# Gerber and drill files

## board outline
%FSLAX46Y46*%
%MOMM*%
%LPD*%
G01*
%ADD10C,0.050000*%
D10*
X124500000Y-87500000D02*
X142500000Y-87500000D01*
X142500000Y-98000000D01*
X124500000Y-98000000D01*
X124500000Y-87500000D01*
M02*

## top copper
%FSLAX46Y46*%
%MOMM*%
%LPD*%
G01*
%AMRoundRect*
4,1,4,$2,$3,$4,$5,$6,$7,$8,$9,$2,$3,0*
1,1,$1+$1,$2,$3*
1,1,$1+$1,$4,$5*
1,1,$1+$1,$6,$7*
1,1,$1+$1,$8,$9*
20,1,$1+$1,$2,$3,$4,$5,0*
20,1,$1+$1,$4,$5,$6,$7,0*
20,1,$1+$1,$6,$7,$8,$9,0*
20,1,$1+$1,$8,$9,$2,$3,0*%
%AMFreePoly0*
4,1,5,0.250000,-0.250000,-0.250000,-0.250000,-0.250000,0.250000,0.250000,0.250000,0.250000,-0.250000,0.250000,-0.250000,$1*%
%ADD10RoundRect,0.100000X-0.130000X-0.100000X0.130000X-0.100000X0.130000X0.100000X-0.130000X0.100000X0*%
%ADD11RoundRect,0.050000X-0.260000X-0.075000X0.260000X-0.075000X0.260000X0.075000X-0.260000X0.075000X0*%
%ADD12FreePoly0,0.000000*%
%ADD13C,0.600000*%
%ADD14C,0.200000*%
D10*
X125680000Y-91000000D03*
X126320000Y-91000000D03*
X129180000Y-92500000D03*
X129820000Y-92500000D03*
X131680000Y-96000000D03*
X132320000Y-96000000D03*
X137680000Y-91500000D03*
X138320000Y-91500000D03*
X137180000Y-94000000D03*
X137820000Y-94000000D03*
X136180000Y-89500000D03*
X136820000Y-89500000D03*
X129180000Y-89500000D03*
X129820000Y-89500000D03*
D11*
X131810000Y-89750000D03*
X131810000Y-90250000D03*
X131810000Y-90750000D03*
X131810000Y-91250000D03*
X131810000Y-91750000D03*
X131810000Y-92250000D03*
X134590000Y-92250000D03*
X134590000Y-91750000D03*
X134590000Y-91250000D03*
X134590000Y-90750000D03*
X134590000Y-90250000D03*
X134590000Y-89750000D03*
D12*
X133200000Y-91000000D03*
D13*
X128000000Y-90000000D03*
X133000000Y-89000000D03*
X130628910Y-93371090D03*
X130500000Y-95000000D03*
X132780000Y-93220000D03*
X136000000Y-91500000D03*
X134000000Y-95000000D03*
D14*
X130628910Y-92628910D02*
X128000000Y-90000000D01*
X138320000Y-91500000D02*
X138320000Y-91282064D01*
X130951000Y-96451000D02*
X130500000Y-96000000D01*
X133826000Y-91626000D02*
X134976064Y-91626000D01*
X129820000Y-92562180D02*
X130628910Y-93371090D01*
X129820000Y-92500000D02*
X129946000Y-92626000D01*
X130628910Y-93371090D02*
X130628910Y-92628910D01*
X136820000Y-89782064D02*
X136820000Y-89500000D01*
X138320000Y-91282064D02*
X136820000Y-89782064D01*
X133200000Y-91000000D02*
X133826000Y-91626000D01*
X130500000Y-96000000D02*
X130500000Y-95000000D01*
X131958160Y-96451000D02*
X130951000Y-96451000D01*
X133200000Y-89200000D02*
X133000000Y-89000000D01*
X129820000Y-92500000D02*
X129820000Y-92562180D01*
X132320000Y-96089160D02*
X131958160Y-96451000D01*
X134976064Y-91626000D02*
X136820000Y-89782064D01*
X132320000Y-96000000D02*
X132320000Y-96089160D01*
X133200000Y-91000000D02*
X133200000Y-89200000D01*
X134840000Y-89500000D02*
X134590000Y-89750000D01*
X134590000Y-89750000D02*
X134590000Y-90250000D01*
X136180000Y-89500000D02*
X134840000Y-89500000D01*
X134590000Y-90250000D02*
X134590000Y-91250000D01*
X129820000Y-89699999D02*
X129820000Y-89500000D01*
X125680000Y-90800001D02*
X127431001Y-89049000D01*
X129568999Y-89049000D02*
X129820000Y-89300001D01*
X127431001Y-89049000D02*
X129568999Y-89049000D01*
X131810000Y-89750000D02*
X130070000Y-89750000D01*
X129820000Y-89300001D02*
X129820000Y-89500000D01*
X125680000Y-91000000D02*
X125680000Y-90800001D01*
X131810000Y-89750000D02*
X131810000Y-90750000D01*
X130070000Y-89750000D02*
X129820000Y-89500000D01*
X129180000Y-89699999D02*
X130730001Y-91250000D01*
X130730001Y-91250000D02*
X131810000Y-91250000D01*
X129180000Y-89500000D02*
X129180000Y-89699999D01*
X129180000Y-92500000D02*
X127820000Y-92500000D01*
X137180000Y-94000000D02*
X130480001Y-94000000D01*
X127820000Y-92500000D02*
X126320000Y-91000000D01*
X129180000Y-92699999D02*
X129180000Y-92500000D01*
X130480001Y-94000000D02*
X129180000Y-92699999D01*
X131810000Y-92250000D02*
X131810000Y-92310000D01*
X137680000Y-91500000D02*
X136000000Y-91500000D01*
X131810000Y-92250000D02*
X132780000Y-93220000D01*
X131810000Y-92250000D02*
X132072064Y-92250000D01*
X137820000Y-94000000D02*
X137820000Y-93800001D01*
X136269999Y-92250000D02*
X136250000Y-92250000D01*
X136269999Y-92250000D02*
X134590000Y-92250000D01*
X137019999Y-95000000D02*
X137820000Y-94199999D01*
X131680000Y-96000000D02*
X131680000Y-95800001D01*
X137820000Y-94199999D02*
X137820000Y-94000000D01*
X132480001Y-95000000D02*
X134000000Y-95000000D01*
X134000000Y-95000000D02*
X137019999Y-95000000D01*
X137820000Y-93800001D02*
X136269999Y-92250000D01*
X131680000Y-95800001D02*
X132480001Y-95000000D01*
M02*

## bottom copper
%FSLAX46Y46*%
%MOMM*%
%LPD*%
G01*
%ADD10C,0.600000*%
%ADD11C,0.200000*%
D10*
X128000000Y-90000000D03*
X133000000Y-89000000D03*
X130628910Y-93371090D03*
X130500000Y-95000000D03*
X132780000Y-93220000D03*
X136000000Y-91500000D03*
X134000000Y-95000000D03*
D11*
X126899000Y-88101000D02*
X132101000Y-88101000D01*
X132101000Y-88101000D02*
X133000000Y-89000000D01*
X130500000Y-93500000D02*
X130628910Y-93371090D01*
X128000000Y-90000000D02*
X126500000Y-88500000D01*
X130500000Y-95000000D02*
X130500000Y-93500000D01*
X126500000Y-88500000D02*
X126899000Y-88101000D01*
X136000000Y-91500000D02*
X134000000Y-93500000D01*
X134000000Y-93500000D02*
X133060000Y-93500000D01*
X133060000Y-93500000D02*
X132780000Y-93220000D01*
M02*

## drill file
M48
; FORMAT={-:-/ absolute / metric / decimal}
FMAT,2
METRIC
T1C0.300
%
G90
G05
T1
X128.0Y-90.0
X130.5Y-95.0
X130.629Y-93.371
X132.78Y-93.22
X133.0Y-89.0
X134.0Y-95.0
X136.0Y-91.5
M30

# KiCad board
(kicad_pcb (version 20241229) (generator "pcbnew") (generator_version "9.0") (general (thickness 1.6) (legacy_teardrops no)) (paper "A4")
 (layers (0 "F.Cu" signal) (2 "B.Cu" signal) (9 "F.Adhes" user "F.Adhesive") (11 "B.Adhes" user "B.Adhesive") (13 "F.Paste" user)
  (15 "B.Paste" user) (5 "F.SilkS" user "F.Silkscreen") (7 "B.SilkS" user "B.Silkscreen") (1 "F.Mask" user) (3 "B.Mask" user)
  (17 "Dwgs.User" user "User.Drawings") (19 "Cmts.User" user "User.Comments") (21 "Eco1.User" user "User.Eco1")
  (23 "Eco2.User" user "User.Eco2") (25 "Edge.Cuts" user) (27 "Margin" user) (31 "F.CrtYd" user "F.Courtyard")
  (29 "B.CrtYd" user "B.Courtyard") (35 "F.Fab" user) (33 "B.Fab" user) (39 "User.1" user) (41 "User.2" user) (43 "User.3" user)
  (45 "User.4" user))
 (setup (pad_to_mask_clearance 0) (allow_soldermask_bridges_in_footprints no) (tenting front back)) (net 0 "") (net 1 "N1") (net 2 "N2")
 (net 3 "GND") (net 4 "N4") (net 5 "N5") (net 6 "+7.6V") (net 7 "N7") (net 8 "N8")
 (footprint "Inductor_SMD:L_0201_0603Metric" (layer "F.Cu") (at 126 91)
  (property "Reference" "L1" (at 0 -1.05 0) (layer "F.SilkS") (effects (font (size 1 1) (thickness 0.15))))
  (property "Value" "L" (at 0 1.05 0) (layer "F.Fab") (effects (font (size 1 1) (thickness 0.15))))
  (pad "" smd roundrect (at -0.345 0) (size 0.318 0.36) (layers "F.Paste") (roundrect_rratio 0.25))
  (pad "" smd roundrect (at 0.345 0) (size 0.318 0.36) (layers "F.Paste") (roundrect_rratio 0.25))
  (pad "1" smd roundrect (at -0.32 0) (size 0.46 0.4) (layers "F.Cu" "F.Mask") (roundrect_rratio 0.25) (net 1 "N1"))
  (pad "2" smd roundrect (at 0.32 0) (size 0.46 0.4) (layers "F.Cu" "F.Mask") (roundrect_rratio 0.25) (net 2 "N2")))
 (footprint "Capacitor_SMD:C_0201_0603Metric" (layer "F.Cu") (at 129.5 92.5)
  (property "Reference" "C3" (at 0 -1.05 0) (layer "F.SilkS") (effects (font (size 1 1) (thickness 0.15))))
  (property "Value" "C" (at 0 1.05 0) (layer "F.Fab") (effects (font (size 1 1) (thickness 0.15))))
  (pad "" smd roundrect (at -0.345 0) (size 0.318 0.36) (layers "F.Paste") (roundrect_rratio 0.25))
  (pad "" smd roundrect (at 0.345 0) (size 0.318 0.36) (layers "F.Paste") (roundrect_rratio 0.25))
  (pad "1" smd roundrect (at -0.32 0) (size 0.46 0.4) (layers "F.Cu" "F.Mask") (roundrect_rratio 0.25) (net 2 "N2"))
  (pad "2" smd roundrect (at 0.32 0) (size 0.46 0.4) (layers "F.Cu" "F.Mask") (roundrect_rratio 0.25) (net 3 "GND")))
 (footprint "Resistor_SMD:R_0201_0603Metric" (layer "F.Cu") (at 132 96)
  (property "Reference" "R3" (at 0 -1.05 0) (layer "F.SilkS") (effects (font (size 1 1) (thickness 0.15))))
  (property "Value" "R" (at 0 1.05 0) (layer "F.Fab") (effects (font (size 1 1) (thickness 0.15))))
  (pad "" smd roundrect (at -0.345 0) (size 0.318 0.36) (layers "F.Paste") (roundrect_rratio 0.25))
  (pad "" smd roundrect (at 0.345 0) (size 0.318 0.36) (layers "F.Paste") (roundrect_rratio 0.25))
  (pad "1" smd roundrect (at -0.32 0) (size 0.46 0.4) (layers "F.Cu" "F.Mask") (roundrect_rratio 0.25) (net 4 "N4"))
  (pad "2" smd roundrect (at 0.32 0) (size 0.46 0.4) (layers "F.Cu" "F.Mask") (roundrect_rratio 0.25) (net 3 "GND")))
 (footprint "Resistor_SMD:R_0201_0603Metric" (layer "F.Cu") (at 138 91.5)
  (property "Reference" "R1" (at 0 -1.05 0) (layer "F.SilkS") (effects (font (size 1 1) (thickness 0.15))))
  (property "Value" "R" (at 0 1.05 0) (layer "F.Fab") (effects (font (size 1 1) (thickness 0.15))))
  (pad "" smd roundrect (at -0.345 0) (size 0.318 0.36) (layers "F.Paste") (roundrect_rratio 0.25))
  (pad "" smd roundrect (at 0.345 0) (size 0.318 0.36) (layers "F.Paste") (roundrect_rratio 0.25))
  (pad "1" smd roundrect (at -0.32 0) (size 0.46 0.4) (layers "F.Cu" "F.Mask") (roundrect_rratio 0.25) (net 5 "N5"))
  (pad "2" smd roundrect (at 0.32 0) (size 0.46 0.4) (layers "F.Cu" "F.Mask") (roundrect_rratio 0.25) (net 3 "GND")))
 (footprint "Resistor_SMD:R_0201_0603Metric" (layer "F.Cu") (at 137.5 94)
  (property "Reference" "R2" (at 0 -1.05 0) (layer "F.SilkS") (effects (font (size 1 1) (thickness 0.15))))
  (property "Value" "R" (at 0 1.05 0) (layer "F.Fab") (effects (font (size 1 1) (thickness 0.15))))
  (pad "" smd roundrect (at -0.345 0) (size 0.318 0.36) (layers "F.Paste") (roundrect_rratio 0.25))
  (pad "" smd roundrect (at 0.345 0) (size 0.318 0.36) (layers "F.Paste") (roundrect_rratio 0.25))
  (pad "1" smd roundrect (at -0.32 0) (size 0.46 0.4) (layers "F.Cu" "F.Mask") (roundrect_rratio 0.25) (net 2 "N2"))
  (pad "2" smd roundrect (at 0.32 0) (size 0.46 0.4) (layers "F.Cu" "F.Mask") (roundrect_rratio 0.25) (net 4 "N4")))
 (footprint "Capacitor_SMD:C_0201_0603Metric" (layer "F.Cu") (at 136.5 89.5)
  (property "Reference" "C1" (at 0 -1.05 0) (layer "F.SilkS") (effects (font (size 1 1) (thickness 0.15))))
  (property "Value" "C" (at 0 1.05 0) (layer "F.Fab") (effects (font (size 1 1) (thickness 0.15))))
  (pad "" smd roundrect (at -0.345 0) (size 0.318 0.36) (layers "F.Paste") (roundrect_rratio 0.25))
  (pad "" smd roundrect (at 0.345 0) (size 0.318 0.36) (layers "F.Paste") (roundrect_rratio 0.25))
  (pad "1" smd roundrect (at -0.32 0) (size 0.46 0.4) (layers "F.Cu" "F.Mask") (roundrect_rratio 0.25) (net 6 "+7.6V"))
  (pad "2" smd roundrect (at 0.32 0) (size 0.46 0.4) (layers "F.Cu" "F.Mask") (roundrect_rratio 0.25) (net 3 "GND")))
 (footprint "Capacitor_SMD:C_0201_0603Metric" (layer "F.Cu") (at 129.5 89.5)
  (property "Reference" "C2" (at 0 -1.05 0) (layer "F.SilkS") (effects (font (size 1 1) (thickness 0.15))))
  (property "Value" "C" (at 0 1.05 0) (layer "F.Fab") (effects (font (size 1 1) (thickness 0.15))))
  (pad "" smd roundrect (at -0.345 0) (size 0.318 0.36) (layers "F.Paste") (roundrect_rratio 0.25))
  (pad "" smd roundrect (at 0.345 0) (size 0.318 0.36) (layers "F.Paste") (roundrect_rratio 0.25))
  (pad "1" smd roundrect (at -0.32 0) (size 0.46 0.4) (layers "F.Cu" "F.Mask") (roundrect_rratio 0.25) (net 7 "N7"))
  (pad "2" smd roundrect (at 0.32 0) (size 0.46 0.4) (layers "F.Cu" "F.Mask") (roundrect_rratio 0.25) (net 1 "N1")))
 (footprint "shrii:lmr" (layer "F.Cu") (at 139.5 94)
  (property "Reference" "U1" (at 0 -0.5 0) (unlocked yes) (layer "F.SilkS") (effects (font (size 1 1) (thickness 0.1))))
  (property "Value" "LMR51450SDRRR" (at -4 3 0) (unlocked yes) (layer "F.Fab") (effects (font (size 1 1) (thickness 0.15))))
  (pad "1" smd roundrect (at -7.69 -4.25) (size 0.62 0.25) (layers "F.Cu" "F.Paste") (roundrect_rratio 0.2) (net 1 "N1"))
  (pad "2" smd roundrect (at -7.69 -3.75) (size 0.62 0.25) (layers "F.Cu" "F.Paste") (roundrect_rratio 0.2) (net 1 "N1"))
  (pad "3" smd roundrect (at -7.69 -3.25) (size 0.62 0.25) (layers "F.Cu" "F.Paste") (roundrect_rratio 0.2) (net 1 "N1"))
  (pad "4" smd roundrect (at -7.69 -2.75) (size 0.62 0.25) (layers "F.Cu" "F.Paste") (roundrect_rratio 0.2) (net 7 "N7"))
  (pad "5" smd roundrect (at -7.69 -2.25) (size 0.62 0.25) (layers "F.Cu" "F.Paste") (roundrect_rratio 0.2) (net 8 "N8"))
  (pad "6" smd roundrect (at -7.69 -1.75) (size 0.62 0.25) (layers "F.Cu" "F.Paste") (roundrect_rratio 0.2) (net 5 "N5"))
  (pad "7" smd roundrect (at -4.91 -1.75) (size 0.62 0.25) (layers "F.Cu" "F.Paste") (roundrect_rratio 0.2) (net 4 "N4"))
  (pad "8" smd roundrect (at -4.91 -2.25) (size 0.62 0.25) (layers "F.Cu" "F.Paste") (roundrect_rratio 0.2) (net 3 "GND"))
  (pad "9" smd roundrect (at -4.91 -2.75) (size 0.62 0.25) (layers "F.Cu" "F.Paste") (roundrect_rratio 0.2) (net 6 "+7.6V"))
  (pad "10" smd roundrect (at -4.91 -3.25) (size 0.62 0.25) (layers "F.Cu" "F.Paste") (roundrect_rratio 0.2) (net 6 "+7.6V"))
  (pad "11" smd roundrect (at -4.91 -3.75) (size 0.62 0.25) (layers "F.Cu" "F.Paste") (roundrect_rratio 0.2) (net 6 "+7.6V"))
  (pad "12" smd roundrect (at -4.91 -4.25) (size 0.62 0.25) (layers "F.Cu" "F.Paste") (roundrect_rratio 0.2) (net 6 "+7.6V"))
  (pad "13" smd custom (at -6.3 -3) (size 0.5 0.5) (layers "F.Cu") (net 3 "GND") (zone_connect 2)
   (options (clearance outline) (anchor rect)) (primitives)))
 (gr_rect (start 124.5 87.5) (end 142.5 98) (stroke (width 0.05) (type default)) (fill no) (layer "Edge.Cuts"))
 (segment (start 130.62891 92.62891) (end 128 90) (width 0.2) (layer "F.Cu") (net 3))
 (segment (start 138.32 91.5) (end 138.32 91.282064) (width 0.2) (layer "F.Cu") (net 3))
 (segment (start 130.951 96.451) (end 130.5 96) (width 0.2) (layer "F.Cu") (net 3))
 (segment (start 133.826 91.626) (end 134.976064 91.626) (width 0.2) (layer "F.Cu") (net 3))
 (segment (start 129.82 92.56218) (end 130.62891 93.37109) (width 0.2) (layer "F.Cu") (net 3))
 (segment (start 129.82 92.5) (end 129.946 92.626) (width 0.2) (layer "F.Cu") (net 3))
 (segment (start 130.62891 93.37109) (end 130.62891 92.62891) (width 0.2) (layer "F.Cu") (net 3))
 (segment (start 136.82 89.782064) (end 136.82 89.5) (width 0.2) (layer "F.Cu") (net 3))
 (segment (start 138.32 91.282064) (end 136.82 89.782064) (width 0.2) (layer "F.Cu") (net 3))
 (segment (start 133.2 91) (end 133.826 91.626) (width 0.2) (layer "F.Cu") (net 3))
 (segment (start 130.5 96) (end 130.5 95) (width 0.2) (layer "F.Cu") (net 3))
 (segment (start 131.95816 96.451) (end 130.951 96.451) (width 0.2) (layer "F.Cu") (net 3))
 (segment (start 133.2 89.2) (end 133 89) (width 0.2) (layer "F.Cu") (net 3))
 (segment (start 129.82 92.5) (end 129.82 92.56218) (width 0.2) (layer "F.Cu") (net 3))
 (segment (start 132.32 96.08916) (end 131.95816 96.451) (width 0.2) (layer "F.Cu") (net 3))
 (segment (start 134.976064 91.626) (end 136.82 89.782064) (width 0.2) (layer "F.Cu") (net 3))
 (segment (start 132.32 96) (end 132.32 96.08916) (width 0.2) (layer "F.Cu") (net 3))
 (segment (start 133.2 91) (end 133.2 89.2) (width 0.2) (layer "F.Cu") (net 3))
 (via (at 128 90) (size 0.6) (drill 0.3) (layers "F.Cu" "B.Cu") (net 3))
 (via (at 133 89) (size 0.6) (drill 0.3) (layers "F.Cu" "B.Cu") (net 3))
 (via (at 130.62891 93.37109) (size 0.6) (drill 0.3) (layers "F.Cu" "B.Cu") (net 3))
 (via (at 130.5 95) (size 0.6) (drill 0.3) (layers "F.Cu" "B.Cu") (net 3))
 (segment (start 126.899 88.101) (end 132.101 88.101) (width 0.2) (layer "B.Cu") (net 3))
 (segment (start 132.101 88.101) (end 133 89) (width 0.2) (layer "B.Cu") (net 3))
 (segment (start 130.5 93.5) (end 130.62891 93.37109) (width 0.2) (layer "B.Cu") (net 3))
 (segment (start 128 90) (end 126.5 88.5) (width 0.2) (layer "B.Cu") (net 3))
 (segment (start 130.5 95) (end 130.5 93.5) (width 0.2) (layer "B.Cu") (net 3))
 (segment (start 126.5 88.5) (end 126.899 88.101) (width 0.2) (layer "B.Cu") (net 3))
 (segment (start 134.84 89.5) (end 134.59 89.75) (width 0.2) (layer "F.Cu") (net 6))
 (segment (start 134.59 89.75) (end 134.59 90.25) (width 0.2) (layer "F.Cu") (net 6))
 (segment (start 136.18 89.5) (end 134.84 89.5) (width 0.2) (layer "F.Cu") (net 6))
 (segment (start 134.59 90.25) (end 134.59 91.25) (width 0.2) (layer "F.Cu") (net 6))
 (segment (start 129.82 89.699999) (end 129.82 89.5) (width 0.2) (layer "F.Cu") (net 1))
 (segment (start 125.68 90.800001) (end 127.431001 89.049) (width 0.2) (layer "F.Cu") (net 1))
 (segment (start 129.568999 89.049) (end 129.82 89.300001) (width 0.2) (layer "F.Cu") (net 1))
 (segment (start 127.431001 89.049) (end 129.568999 89.049) (width 0.2) (layer "F.Cu") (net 1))
 (segment (start 131.81 89.75) (end 130.07 89.75) (width 0.2) (layer "F.Cu") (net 1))
 (segment (start 129.82 89.300001) (end 129.82 89.5) (width 0.2) (layer "F.Cu") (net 1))
 (segment (start 125.68 91) (end 125.68 90.800001) (width 0.2) (layer "F.Cu") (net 1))
 (segment (start 131.81 89.75) (end 131.81 90.75) (width 0.2) (layer "F.Cu") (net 1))
 (segment (start 130.07 89.75) (end 129.82 89.5) (width 0.2) (layer "F.Cu") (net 1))
 (segment (start 129.18 89.699999) (end 130.730001 91.25) (width 0.2) (layer "F.Cu") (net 7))
 (segment (start 130.730001 91.25) (end 131.81 91.25) (width 0.2) (layer "F.Cu") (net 7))
 (segment (start 129.18 89.5) (end 129.18 89.699999) (width 0.2) (layer "F.Cu") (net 7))
 (segment (start 129.18 92.5) (end 127.82 92.5) (width 0.2) (layer "F.Cu") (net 2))
 (segment (start 137.18 94) (end 130.480001 94) (width 0.2) (layer "F.Cu") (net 2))
 (segment (start 127.82 92.5) (end 126.32 91) (width 0.2) (layer "F.Cu") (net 2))
 (segment (start 129.18 92.699999) (end 129.18 92.5) (width 0.2) (layer "F.Cu") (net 2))
 (segment (start 130.480001 94) (end 129.18 92.699999) (width 0.2) (layer "F.Cu") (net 2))
 (segment (start 131.81 92.25) (end 131.81 92.31) (width 0.2) (layer "F.Cu") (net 5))
 (segment (start 137.68 91.5) (end 136 91.5) (width 0.2) (layer "F.Cu") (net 5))
 (segment (start 131.81 92.25) (end 132.78 93.22) (width 0.2) (layer "F.Cu") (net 5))
 (segment (start 131.81 92.25) (end 132.072064 92.25) (width 0.2) (layer "F.Cu") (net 5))
 (via (at 132.78 93.22) (size 0.6) (drill 0.3) (layers "F.Cu" "B.Cu") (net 5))
 (via (at 136 91.5) (size 0.6) (drill 0.3) (layers "F.Cu" "B.Cu") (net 5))
 (segment (start 136 91.5) (end 134 93.5) (width 0.2) (layer "B.Cu") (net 5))
 (segment (start 134 93.5) (end 133.06 93.5) (width 0.2) (layer "B.Cu") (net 5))
 (segment (start 133.06 93.5) (end 132.78 93.22) (width 0.2) (layer "B.Cu") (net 5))
 (segment (start 137.82 94) (end 137.82 93.800001) (width 0.2) (layer "F.Cu") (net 4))
 (segment (start 136.269999 92.25) (end 136.25 92.25) (width 0.2) (layer "F.Cu") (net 4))
 (segment (start 136.269999 92.25) (end 134.59 92.25) (width 0.2) (layer "F.Cu") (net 4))
 (segment (start 137.019999 95) (end 137.82 94.199999) (width 0.2) (layer "F.Cu") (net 4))
 (segment (start 131.68 96) (end 131.68 95.800001) (width 0.2) (layer "F.Cu") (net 4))
 (segment (start 137.82 94.199999) (end 137.82 94) (width 0.2) (layer "F.Cu") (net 4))
 (segment (start 132.480001 95) (end 134 95) (width 0.2) (layer "F.Cu") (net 4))
 (segment (start 134 95) (end 137.019999 95) (width 0.2) (layer "F.Cu") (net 4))
 (segment (start 137.82 93.800001) (end 136.269999 92.25) (width 0.2) (layer "F.Cu") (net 4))
 (segment (start 131.68 95.800001) (end 132.480001 95) (width 0.2) (layer "F.Cu") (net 4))
 (via (at 134 95) (size 0.6) (drill 0.3) (layers "F.Cu" "B.Cu") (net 4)))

